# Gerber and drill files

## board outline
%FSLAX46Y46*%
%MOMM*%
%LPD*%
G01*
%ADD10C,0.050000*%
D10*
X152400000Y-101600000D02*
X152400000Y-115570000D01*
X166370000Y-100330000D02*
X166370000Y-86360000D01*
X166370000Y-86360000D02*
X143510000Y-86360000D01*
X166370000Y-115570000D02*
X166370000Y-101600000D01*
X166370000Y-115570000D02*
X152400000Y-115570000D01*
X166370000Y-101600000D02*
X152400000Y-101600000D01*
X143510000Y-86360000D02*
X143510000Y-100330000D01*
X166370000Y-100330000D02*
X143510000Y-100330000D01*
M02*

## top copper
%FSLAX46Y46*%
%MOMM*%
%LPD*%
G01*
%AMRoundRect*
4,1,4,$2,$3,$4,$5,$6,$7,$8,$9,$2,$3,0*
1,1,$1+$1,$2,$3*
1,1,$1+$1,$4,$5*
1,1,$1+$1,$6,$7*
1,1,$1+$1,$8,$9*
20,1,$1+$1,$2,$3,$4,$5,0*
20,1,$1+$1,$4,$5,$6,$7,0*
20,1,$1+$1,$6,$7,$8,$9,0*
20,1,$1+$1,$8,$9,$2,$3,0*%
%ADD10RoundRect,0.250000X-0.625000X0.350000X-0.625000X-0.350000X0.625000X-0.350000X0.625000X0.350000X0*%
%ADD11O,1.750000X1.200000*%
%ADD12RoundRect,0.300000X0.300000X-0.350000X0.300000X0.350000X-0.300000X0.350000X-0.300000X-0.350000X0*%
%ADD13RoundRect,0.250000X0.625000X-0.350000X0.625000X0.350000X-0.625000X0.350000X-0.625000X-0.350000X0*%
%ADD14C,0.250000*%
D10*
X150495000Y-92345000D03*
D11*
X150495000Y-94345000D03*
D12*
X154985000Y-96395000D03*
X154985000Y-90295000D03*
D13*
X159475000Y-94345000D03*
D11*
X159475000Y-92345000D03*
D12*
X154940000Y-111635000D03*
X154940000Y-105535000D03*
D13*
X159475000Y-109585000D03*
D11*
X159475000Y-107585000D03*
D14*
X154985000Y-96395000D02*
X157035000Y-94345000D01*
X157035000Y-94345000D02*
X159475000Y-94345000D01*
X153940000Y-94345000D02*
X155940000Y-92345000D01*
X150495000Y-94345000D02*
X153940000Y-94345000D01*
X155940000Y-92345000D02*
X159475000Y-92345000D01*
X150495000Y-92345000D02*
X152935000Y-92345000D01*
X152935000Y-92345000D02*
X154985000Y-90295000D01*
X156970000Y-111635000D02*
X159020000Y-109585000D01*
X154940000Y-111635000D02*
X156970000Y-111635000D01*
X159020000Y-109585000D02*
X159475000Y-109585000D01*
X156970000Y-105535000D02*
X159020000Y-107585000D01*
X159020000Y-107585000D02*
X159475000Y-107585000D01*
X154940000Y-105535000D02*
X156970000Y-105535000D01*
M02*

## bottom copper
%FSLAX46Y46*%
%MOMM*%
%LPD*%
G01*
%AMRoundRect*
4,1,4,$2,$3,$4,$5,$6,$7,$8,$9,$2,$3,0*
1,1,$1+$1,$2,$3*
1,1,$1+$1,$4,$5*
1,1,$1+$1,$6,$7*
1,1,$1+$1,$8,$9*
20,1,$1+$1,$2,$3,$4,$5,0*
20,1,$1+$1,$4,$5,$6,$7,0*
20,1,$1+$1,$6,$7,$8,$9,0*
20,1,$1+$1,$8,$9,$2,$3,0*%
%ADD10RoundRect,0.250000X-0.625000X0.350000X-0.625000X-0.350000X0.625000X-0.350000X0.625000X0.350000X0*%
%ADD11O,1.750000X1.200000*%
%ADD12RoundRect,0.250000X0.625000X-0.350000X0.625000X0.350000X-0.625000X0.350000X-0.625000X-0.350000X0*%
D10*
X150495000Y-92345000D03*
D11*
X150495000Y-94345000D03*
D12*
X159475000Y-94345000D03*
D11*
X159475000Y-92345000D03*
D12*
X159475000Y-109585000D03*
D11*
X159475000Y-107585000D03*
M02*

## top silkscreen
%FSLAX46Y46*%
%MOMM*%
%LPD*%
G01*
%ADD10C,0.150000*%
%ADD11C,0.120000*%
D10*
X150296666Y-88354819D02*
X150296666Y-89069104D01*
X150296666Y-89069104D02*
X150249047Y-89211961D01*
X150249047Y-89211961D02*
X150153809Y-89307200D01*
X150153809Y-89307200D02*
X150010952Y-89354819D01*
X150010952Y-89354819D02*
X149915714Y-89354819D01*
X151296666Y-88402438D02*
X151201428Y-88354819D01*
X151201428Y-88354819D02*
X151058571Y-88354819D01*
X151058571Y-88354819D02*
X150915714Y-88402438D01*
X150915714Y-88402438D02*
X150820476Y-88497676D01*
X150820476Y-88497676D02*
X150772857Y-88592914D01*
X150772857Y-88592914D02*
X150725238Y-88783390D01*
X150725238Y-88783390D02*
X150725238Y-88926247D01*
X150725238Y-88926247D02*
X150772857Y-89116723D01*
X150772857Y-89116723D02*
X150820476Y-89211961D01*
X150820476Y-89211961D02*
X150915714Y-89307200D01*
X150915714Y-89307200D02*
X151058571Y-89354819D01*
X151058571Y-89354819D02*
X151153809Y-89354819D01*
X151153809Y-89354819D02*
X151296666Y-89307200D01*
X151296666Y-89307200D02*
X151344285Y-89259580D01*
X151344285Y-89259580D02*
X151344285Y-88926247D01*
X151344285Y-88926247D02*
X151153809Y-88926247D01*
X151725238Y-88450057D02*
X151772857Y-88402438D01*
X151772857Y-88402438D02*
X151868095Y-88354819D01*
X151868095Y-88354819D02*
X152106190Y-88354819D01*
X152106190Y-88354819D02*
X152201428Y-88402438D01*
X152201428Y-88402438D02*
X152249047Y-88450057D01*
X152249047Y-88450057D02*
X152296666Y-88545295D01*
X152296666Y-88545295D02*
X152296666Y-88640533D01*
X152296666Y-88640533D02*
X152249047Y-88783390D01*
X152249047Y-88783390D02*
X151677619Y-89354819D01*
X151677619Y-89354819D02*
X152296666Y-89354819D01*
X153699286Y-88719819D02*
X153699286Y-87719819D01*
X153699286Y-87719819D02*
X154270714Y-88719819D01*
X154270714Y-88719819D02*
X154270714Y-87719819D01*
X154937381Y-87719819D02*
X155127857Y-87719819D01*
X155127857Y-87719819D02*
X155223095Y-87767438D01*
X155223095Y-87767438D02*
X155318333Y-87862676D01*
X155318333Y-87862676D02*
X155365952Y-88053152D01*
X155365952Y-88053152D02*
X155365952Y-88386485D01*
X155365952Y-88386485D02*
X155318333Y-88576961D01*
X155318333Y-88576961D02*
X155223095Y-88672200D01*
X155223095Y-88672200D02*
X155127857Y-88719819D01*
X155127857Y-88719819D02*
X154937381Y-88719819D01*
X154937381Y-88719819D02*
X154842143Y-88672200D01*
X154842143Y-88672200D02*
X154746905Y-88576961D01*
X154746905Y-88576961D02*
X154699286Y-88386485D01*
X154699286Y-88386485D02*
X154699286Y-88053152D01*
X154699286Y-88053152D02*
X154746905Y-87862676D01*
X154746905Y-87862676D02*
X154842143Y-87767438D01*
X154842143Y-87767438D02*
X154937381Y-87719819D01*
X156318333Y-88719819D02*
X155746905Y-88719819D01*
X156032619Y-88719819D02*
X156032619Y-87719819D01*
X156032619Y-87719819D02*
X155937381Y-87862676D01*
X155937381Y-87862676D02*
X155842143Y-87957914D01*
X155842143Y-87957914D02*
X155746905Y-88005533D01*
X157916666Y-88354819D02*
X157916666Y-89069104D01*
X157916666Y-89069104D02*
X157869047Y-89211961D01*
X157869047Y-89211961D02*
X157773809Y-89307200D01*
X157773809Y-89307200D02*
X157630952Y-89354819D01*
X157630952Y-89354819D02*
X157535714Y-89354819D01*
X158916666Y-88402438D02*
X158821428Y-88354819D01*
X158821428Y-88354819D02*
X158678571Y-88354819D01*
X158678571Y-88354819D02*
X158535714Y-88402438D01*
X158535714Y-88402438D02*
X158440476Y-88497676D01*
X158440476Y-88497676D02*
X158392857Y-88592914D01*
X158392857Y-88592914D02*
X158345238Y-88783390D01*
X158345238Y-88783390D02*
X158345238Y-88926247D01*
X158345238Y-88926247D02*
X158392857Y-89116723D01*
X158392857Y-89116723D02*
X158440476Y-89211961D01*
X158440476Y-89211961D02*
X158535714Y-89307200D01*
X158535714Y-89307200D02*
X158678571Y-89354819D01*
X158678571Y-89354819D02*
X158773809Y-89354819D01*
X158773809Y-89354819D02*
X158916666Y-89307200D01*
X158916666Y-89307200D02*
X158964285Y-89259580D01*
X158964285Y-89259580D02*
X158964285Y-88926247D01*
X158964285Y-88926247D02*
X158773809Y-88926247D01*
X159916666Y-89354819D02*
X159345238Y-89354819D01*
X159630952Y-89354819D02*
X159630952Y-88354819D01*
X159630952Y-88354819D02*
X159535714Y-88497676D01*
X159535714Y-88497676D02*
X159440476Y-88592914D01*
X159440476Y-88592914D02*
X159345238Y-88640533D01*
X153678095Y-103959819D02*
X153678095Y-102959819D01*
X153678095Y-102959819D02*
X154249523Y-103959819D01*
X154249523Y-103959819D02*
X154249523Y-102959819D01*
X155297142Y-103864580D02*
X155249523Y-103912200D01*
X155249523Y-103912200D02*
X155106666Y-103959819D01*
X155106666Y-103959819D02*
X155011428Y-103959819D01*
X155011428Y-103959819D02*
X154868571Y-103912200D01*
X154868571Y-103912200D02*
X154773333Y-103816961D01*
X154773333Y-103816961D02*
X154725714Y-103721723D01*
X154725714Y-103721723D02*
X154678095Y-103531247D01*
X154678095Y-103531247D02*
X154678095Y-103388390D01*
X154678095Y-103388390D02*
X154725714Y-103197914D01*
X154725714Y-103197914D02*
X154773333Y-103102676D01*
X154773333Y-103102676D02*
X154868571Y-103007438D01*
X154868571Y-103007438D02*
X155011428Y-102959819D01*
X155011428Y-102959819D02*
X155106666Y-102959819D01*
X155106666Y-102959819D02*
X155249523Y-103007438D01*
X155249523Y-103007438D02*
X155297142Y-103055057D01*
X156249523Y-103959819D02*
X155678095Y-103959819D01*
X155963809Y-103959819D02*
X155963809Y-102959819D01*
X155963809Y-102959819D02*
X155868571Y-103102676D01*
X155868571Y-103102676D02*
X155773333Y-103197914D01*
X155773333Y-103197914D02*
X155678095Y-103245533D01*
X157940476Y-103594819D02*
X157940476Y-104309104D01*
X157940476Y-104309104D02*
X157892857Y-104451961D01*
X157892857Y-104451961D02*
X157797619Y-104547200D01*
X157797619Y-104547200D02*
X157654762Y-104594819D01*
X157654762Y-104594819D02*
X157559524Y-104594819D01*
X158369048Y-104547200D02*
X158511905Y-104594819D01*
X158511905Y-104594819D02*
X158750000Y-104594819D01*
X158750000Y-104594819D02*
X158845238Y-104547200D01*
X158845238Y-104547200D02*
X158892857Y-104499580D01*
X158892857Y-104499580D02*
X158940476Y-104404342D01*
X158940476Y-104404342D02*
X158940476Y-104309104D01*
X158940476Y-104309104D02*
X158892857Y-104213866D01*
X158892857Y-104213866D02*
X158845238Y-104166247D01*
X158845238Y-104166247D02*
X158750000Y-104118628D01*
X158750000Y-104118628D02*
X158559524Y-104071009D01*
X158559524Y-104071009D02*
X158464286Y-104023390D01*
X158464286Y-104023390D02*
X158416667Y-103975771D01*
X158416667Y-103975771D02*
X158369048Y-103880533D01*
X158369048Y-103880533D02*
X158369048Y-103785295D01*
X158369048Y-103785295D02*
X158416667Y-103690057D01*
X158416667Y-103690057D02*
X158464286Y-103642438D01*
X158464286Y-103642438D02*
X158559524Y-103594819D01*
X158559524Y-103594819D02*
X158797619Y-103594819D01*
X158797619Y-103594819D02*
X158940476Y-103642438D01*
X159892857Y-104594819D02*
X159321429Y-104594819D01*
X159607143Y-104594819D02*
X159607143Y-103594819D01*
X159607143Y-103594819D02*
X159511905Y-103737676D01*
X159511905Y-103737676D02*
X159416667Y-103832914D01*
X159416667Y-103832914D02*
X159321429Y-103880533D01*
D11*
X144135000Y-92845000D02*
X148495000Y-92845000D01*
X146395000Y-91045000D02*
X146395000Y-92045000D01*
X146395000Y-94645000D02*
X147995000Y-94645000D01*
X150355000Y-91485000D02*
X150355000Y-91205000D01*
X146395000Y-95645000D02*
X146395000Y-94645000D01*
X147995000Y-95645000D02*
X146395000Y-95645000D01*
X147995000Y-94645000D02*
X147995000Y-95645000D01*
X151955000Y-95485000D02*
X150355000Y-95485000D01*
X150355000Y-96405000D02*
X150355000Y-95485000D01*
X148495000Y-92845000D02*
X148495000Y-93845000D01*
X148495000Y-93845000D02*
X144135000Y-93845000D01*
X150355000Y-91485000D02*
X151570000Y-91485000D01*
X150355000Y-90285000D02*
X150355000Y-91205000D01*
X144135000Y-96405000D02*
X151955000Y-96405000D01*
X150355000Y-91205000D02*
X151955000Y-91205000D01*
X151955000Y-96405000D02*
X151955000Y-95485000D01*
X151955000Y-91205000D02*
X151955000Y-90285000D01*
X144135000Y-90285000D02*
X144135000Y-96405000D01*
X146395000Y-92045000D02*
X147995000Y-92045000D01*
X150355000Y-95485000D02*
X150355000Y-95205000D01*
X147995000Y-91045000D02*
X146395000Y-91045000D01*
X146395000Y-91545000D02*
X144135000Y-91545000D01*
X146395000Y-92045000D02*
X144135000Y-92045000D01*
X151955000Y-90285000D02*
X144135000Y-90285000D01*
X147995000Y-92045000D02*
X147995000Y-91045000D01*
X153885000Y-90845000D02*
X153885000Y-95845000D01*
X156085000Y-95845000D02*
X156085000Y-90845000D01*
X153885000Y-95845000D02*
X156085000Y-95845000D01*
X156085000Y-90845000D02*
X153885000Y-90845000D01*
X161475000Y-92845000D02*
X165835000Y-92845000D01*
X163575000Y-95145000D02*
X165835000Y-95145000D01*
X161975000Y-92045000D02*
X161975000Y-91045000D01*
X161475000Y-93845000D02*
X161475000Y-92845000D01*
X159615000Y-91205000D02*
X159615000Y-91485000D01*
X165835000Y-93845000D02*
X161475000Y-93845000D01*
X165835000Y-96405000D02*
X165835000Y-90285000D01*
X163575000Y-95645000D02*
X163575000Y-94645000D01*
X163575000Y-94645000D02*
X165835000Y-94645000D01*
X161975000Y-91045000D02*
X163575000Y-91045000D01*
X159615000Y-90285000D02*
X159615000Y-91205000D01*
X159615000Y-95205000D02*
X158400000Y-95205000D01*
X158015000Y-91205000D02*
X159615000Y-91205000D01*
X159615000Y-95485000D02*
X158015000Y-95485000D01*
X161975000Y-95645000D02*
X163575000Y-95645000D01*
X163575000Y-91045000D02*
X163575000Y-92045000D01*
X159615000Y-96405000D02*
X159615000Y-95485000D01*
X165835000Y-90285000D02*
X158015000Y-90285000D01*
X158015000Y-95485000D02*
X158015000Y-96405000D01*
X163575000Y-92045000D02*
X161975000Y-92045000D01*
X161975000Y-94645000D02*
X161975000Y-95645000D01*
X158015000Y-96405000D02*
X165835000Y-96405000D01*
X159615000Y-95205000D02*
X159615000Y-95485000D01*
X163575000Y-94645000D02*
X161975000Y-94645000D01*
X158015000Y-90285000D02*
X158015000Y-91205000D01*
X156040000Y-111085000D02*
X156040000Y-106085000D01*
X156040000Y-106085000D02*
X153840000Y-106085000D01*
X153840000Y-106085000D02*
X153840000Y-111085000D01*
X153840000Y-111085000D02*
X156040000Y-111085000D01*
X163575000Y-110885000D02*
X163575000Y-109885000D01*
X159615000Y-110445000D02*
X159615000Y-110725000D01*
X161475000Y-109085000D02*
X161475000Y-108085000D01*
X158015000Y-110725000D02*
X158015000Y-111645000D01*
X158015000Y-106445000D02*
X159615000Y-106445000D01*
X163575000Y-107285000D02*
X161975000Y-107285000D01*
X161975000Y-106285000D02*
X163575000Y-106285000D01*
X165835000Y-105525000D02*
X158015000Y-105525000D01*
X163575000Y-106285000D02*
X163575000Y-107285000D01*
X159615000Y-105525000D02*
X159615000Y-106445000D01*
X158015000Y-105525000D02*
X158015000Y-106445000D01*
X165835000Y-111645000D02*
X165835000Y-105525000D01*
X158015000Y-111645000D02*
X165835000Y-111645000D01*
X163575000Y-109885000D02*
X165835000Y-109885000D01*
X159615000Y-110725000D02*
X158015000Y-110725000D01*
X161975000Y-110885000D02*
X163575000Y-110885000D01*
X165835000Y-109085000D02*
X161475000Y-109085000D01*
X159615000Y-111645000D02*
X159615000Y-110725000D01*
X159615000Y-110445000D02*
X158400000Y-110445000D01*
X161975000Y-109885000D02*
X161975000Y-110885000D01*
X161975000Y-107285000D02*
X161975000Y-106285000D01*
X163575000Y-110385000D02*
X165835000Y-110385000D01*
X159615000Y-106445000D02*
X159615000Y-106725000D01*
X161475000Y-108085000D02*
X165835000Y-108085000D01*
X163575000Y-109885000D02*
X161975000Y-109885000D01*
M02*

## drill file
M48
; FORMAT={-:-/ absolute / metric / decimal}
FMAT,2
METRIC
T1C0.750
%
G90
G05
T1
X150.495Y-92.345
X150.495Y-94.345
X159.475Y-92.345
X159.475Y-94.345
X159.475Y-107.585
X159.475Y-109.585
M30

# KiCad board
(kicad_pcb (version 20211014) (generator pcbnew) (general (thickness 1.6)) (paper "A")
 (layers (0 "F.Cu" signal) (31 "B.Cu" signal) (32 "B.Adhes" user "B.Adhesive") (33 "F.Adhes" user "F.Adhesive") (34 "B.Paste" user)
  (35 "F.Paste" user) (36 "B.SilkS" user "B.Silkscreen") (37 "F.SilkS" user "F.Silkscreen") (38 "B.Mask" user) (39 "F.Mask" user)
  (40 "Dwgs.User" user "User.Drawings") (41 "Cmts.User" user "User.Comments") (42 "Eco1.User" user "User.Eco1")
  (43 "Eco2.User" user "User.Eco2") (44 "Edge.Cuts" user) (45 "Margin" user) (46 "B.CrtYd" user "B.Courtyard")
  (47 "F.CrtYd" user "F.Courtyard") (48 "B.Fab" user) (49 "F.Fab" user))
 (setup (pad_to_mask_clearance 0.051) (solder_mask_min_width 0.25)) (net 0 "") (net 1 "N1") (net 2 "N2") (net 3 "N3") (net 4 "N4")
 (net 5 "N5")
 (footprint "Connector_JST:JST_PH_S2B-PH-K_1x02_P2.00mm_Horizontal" (layer "F.Cu") (at 150.495 92.345 -90)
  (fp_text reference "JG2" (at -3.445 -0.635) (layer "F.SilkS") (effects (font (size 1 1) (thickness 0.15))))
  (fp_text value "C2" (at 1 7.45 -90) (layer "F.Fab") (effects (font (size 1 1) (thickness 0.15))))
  (fp_line (start 0.5 6.36) (end 0.5 2) (layer "F.SilkS") (width 0.12))
  (fp_line (start -1.3 4.1) (end -0.3 4.1) (layer "F.SilkS") (width 0.12))
  (fp_line (start 2.3 4.1) (end 2.3 2.5) (layer "F.SilkS") (width 0.12))
  (fp_line (start -0.86 0.14) (end -1.14 0.14) (layer "F.SilkS") (width 0.12))
  (fp_line (start 3.3 4.1) (end 2.3 4.1) (layer "F.SilkS") (width 0.12))
  (fp_line (start 3.3 2.5) (end 3.3 4.1) (layer "F.SilkS") (width 0.12))
  (fp_line (start 2.3 2.5) (end 3.3 2.5) (layer "F.SilkS") (width 0.12))
  (fp_line (start 3.14 -1.46) (end 3.14 0.14) (layer "F.SilkS") (width 0.12))
  (fp_line (start 4.06 0.14) (end 3.14 0.14) (layer "F.SilkS") (width 0.12))
  (fp_line (start 0.5 2) (end 1.5 2) (layer "F.SilkS") (width 0.12))
  (fp_line (start 1.5 2) (end 1.5 6.36) (layer "F.SilkS") (width 0.12))
  (fp_line (start -0.86 0.14) (end -0.86 -1.075) (layer "F.SilkS") (width 0.12))
  (fp_line (start -2.06 0.14) (end -1.14 0.14) (layer "F.SilkS") (width 0.12))
  (fp_line (start 4.06 6.36) (end 4.06 -1.46) (layer "F.SilkS") (width 0.12))
  (fp_line (start -1.14 0.14) (end -1.14 -1.46) (layer "F.SilkS") (width 0.12))
  (fp_line (start 4.06 -1.46) (end 3.14 -1.46) (layer "F.SilkS") (width 0.12))
  (fp_line (start -1.14 -1.46) (end -2.06 -1.46) (layer "F.SilkS") (width 0.12))
  (fp_line (start -2.06 6.36) (end 4.06 6.36) (layer "F.SilkS") (width 0.12))
  (fp_line (start -0.3 4.1) (end -0.3 2.5) (layer "F.SilkS") (width 0.12))
  (fp_line (start 3.14 0.14) (end 2.86 0.14) (layer "F.SilkS") (width 0.12))
  (fp_line (start -1.3 2.5) (end -1.3 4.1) (layer "F.SilkS") (width 0.12))
  (fp_line (start -0.8 4.1) (end -0.8 6.36) (layer "F.SilkS") (width 0.12))
  (fp_line (start -0.3 4.1) (end -0.3 6.36) (layer "F.SilkS") (width 0.12))
  (fp_line (start -2.06 -1.46) (end -2.06 6.36) (layer "F.SilkS") (width 0.12))
  (fp_line (start -0.3 2.5) (end -1.3 2.5) (layer "F.SilkS") (width 0.12))
  (pad "1" thru_hole roundrect (at 0 0 270) (size 1.2 1.75) (drill 0.75) (layers *.Cu *.Mask) (roundrect_rratio 0.2083333333) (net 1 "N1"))
  (pad "2" thru_hole oval (at 2 0 270) (size 1.2 1.75) (drill 0.75) (layers *.Cu *.Mask) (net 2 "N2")))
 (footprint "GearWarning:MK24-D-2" (layer "F.Cu") (at 154.985 93.345 90)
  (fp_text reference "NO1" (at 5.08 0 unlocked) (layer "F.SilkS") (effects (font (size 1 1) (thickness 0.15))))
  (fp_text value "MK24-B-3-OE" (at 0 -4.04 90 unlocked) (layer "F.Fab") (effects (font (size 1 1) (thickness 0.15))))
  (fp_line (start 2.5 -1.1) (end -2.5 -1.1) (layer "F.SilkS") (width 0.12))
  (fp_line (start -2.5 1.1) (end 2.5 1.1) (layer "F.SilkS") (width 0.12))
  (fp_line (start -2.5 -1.1) (end -2.5 1.1) (layer "F.SilkS") (width 0.12))
  (fp_line (start 2.5 1.1) (end 2.5 -1.1) (layer "F.SilkS") (width 0.12))
  (pad "1" smd roundrect (at -3.05 0 90) (size 1.3 1.2) (layers "F.Cu" "F.Paste" "F.Mask") (roundrect_rratio 0.25) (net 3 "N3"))
  (pad "2" smd roundrect (at 3.05 0 90) (size 1.3 1.2) (layers "F.Cu" "F.Paste" "F.Mask") (roundrect_rratio 0.25) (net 1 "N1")))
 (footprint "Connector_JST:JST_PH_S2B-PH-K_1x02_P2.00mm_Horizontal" (layer "F.Cu") (at 159.475 94.345 90)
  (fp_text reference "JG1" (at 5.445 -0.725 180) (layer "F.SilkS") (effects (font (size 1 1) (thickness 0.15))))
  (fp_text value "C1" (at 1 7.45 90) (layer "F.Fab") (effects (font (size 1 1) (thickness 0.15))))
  (fp_line (start 1.5 2) (end 1.5 6.36) (layer "F.SilkS") (width 0.12))
  (fp_line (start -0.8 4.1) (end -0.8 6.36) (layer "F.SilkS") (width 0.12))
  (fp_line (start 2.3 2.5) (end 3.3 2.5) (layer "F.SilkS") (width 0.12))
  (fp_line (start 0.5 2) (end 1.5 2) (layer "F.SilkS") (width 0.12))
  (fp_line (start 3.14 0.14) (end 2.86 0.14) (layer "F.SilkS") (width 0.12))
  (fp_line (start 0.5 6.36) (end 0.5 2) (layer "F.SilkS") (width 0.12))
  (fp_line (start -2.06 6.36) (end 4.06 6.36) (layer "F.SilkS") (width 0.12))
  (fp_line (start -1.3 4.1) (end -0.3 4.1) (layer "F.SilkS") (width 0.12))
  (fp_line (start -0.3 4.1) (end -0.3 6.36) (layer "F.SilkS") (width 0.12))
  (fp_line (start 3.3 2.5) (end 3.3 4.1) (layer "F.SilkS") (width 0.12))
  (fp_line (start 4.06 0.14) (end 3.14 0.14) (layer "F.SilkS") (width 0.12))
  (fp_line (start -0.86 0.14) (end -0.86 -1.075) (layer "F.SilkS") (width 0.12))
  (fp_line (start 3.14 -1.46) (end 3.14 0.14) (layer "F.SilkS") (width 0.12))
  (fp_line (start -1.14 0.14) (end -1.14 -1.46) (layer "F.SilkS") (width 0.12))
  (fp_line (start -1.3 2.5) (end -1.3 4.1) (layer "F.SilkS") (width 0.12))
  (fp_line (start 3.3 4.1) (end 2.3 4.1) (layer "F.SilkS") (width 0.12))
  (fp_line (start -2.06 0.14) (end -1.14 0.14) (layer "F.SilkS") (width 0.12))
  (fp_line (start 4.06 6.36) (end 4.06 -1.46) (layer "F.SilkS") (width 0.12))
  (fp_line (start -1.14 -1.46) (end -2.06 -1.46) (layer "F.SilkS") (width 0.12))
  (fp_line (start 2.3 4.1) (end 2.3 2.5) (layer "F.SilkS") (width 0.12))
  (fp_line (start -0.3 2.5) (end -1.3 2.5) (layer "F.SilkS") (width 0.12))
  (fp_line (start -2.06 -1.46) (end -2.06 6.36) (layer "F.SilkS") (width 0.12))
  (fp_line (start -0.86 0.14) (end -1.14 0.14) (layer "F.SilkS") (width 0.12))
  (fp_line (start -0.3 4.1) (end -0.3 2.5) (layer "F.SilkS") (width 0.12))
  (fp_line (start 4.06 -1.46) (end 3.14 -1.46) (layer "F.SilkS") (width 0.12))
  (pad "1" thru_hole roundrect (at 0 0 90) (size 1.2 1.75) (drill 0.75) (layers *.Cu *.Mask) (roundrect_rratio 0.2083333333) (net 3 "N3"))
  (pad "2" thru_hole oval (at 2 0 90) (size 1.2 1.75) (drill 0.75) (layers *.Cu *.Mask) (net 2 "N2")))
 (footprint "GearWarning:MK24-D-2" (layer "F.Cu") (at 154.94 108.585 90)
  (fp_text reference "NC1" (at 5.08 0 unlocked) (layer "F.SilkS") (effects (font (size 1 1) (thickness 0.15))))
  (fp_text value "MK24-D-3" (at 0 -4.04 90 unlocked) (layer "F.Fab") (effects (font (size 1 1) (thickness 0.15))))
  (fp_line (start -2.5 1.1) (end 2.5 1.1) (layer "F.SilkS") (width 0.12))
  (fp_line (start 2.5 1.1) (end 2.5 -1.1) (layer "F.SilkS") (width 0.12))
  (fp_line (start 2.5 -1.1) (end -2.5 -1.1) (layer "F.SilkS") (width 0.12))
  (fp_line (start -2.5 -1.1) (end -2.5 1.1) (layer "F.SilkS") (width 0.12))
  (pad "1" smd roundrect (at -3.05 0 90) (size 1.3 1.2) (layers "F.Cu" "F.Paste" "F.Mask") (roundrect_rratio 0.25) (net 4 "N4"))
  (pad "2" smd roundrect (at 3.05 0 90) (size 1.3 1.2) (layers "F.Cu" "F.Paste" "F.Mask") (roundrect_rratio 0.25) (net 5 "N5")))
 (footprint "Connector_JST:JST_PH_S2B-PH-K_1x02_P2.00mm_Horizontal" (layer "F.Cu") (at 159.475 109.585 90)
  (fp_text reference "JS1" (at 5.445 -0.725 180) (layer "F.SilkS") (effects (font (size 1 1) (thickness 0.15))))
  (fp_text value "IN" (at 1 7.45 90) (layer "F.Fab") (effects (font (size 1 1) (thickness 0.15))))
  (fp_line (start -1.3 4.1) (end -0.3 4.1) (layer "F.SilkS") (width 0.12))
  (fp_line (start -0.86 0.14) (end -1.14 0.14) (layer "F.SilkS") (width 0.12))
  (fp_line (start 0.5 2) (end 1.5 2) (layer "F.SilkS") (width 0.12))
  (fp_line (start -1.14 -1.46) (end -2.06 -1.46) (layer "F.SilkS") (width 0.12))
  (fp_line (start 3.14 -1.46) (end 3.14 0.14) (layer "F.SilkS") (width 0.12))
  (fp_line (start 2.3 4.1) (end 2.3 2.5) (layer "F.SilkS") (width 0.12))
  (fp_line (start 3.3 2.5) (end 3.3 4.1) (layer "F.SilkS") (width 0.12))
  (fp_line (start 4.06 6.36) (end 4.06 -1.46) (layer "F.SilkS") (width 0.12))
  (fp_line (start 3.3 4.1) (end 2.3 4.1) (layer "F.SilkS") (width 0.12))
  (fp_line (start 4.06 0.14) (end 3.14 0.14) (layer "F.SilkS") (width 0.12))
  (fp_line (start 4.06 -1.46) (end 3.14 -1.46) (layer "F.SilkS") (width 0.12))
  (fp_line (start -2.06 6.36) (end 4.06 6.36) (layer "F.SilkS") (width 0.12))
  (fp_line (start -2.06 -1.46) (end -2.06 6.36) (layer "F.SilkS") (width 0.12))
  (fp_line (start -0.3 4.1) (end -0.3 6.36) (layer "F.SilkS") (width 0.12))
  (fp_line (start -1.14 0.14) (end -1.14 -1.46) (layer "F.SilkS") (width 0.12))
  (fp_line (start -1.3 2.5) (end -1.3 4.1) (layer "F.SilkS") (width 0.12))
  (fp_line (start 0.5 6.36) (end 0.5 2) (layer "F.SilkS") (width 0.12))
  (fp_line (start -2.06 0.14) (end -1.14 0.14) (layer "F.SilkS") (width 0.12))
  (fp_line (start -0.86 0.14) (end -0.86 -1.075) (layer "F.SilkS") (width 0.12))
  (fp_line (start -0.3 2.5) (end -1.3 2.5) (layer "F.SilkS") (width 0.12))
  (fp_line (start 2.3 2.5) (end 3.3 2.5) (layer "F.SilkS") (width 0.12))
  (fp_line (start -0.8 4.1) (end -0.8 6.36) (layer "F.SilkS") (width 0.12))
  (fp_line (start 3.14 0.14) (end 2.86 0.14) (layer "F.SilkS") (width 0.12))
  (fp_line (start 1.5 2) (end 1.5 6.36) (layer "F.SilkS") (width 0.12))
  (fp_line (start -0.3 4.1) (end -0.3 2.5) (layer "F.SilkS") (width 0.12))
  (pad "1" thru_hole roundrect (at 0 0 90) (size 1.2 1.75) (drill 0.75) (layers *.Cu *.Mask) (roundrect_rratio 0.2083333333) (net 4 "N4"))
  (pad "2" thru_hole oval (at 2 0 90) (size 1.2 1.75) (drill 0.75) (layers *.Cu *.Mask) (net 5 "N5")))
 (gr_line (start 152.4 101.6) (end 152.4 115.57) (layer "Edge.Cuts") (width 0.05))
 (gr_line (start 166.37 100.33) (end 166.37 86.36) (layer "Edge.Cuts") (width 0.05))
 (gr_line (start 166.37 86.36) (end 143.51 86.36) (layer "Edge.Cuts") (width 0.05))
 (gr_line (start 166.37 115.57) (end 166.37 101.6) (layer "Edge.Cuts") (width 0.05))
 (gr_line (start 166.37 115.57) (end 152.4 115.57) (layer "Edge.Cuts") (width 0.05))
 (gr_line (start 166.37 101.6) (end 152.4 101.6) (layer "Edge.Cuts") (width 0.05))
 (gr_line (start 143.51 86.36) (end 143.51 100.33) (layer "Edge.Cuts") (width 0.05))
 (gr_line (start 166.37 100.33) (end 143.51 100.33) (layer "Edge.Cuts") (width 0.05))
 (segment (start 154.985 96.395) (end 157.035 94.345) (width 0.25) (layer "F.Cu") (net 3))
 (segment (start 157.035 94.345) (end 159.475 94.345) (width 0.25) (layer "F.Cu") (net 3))
 (segment (start 153.94 94.345) (end 155.94 92.345) (width 0.25) (layer "F.Cu") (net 2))
 (segment (start 150.495 94.345) (end 153.94 94.345) (width 0.25) (layer "F.Cu") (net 2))
 (segment (start 155.94 92.345) (end 159.475 92.345) (width 0.25) (layer "F.Cu") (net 2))
 (segment (start 150.495 92.345) (end 152.935 92.345) (width 0.25) (layer "F.Cu") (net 1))
 (segment (start 152.935 92.345) (end 154.985 90.295) (width 0.25) (layer "F.Cu") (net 1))
 (segment (start 156.97 111.635) (end 159.02 109.585) (width 0.25) (layer "F.Cu") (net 4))
 (segment (start 154.94 111.635) (end 156.97 111.635) (width 0.25) (layer "F.Cu") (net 4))
 (segment (start 159.02 109.585) (end 159.475 109.585) (width 0.25) (layer "F.Cu") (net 4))
 (segment (start 156.97 105.535) (end 159.02 107.585) (width 0.25) (layer "F.Cu") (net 5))
 (segment (start 159.02 107.585) (end 159.475 107.585) (width 0.25) (layer "F.Cu") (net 5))
 (segment (start 154.94 105.535) (end 156.97 105.535) (width 0.25) (layer "F.Cu") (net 5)))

